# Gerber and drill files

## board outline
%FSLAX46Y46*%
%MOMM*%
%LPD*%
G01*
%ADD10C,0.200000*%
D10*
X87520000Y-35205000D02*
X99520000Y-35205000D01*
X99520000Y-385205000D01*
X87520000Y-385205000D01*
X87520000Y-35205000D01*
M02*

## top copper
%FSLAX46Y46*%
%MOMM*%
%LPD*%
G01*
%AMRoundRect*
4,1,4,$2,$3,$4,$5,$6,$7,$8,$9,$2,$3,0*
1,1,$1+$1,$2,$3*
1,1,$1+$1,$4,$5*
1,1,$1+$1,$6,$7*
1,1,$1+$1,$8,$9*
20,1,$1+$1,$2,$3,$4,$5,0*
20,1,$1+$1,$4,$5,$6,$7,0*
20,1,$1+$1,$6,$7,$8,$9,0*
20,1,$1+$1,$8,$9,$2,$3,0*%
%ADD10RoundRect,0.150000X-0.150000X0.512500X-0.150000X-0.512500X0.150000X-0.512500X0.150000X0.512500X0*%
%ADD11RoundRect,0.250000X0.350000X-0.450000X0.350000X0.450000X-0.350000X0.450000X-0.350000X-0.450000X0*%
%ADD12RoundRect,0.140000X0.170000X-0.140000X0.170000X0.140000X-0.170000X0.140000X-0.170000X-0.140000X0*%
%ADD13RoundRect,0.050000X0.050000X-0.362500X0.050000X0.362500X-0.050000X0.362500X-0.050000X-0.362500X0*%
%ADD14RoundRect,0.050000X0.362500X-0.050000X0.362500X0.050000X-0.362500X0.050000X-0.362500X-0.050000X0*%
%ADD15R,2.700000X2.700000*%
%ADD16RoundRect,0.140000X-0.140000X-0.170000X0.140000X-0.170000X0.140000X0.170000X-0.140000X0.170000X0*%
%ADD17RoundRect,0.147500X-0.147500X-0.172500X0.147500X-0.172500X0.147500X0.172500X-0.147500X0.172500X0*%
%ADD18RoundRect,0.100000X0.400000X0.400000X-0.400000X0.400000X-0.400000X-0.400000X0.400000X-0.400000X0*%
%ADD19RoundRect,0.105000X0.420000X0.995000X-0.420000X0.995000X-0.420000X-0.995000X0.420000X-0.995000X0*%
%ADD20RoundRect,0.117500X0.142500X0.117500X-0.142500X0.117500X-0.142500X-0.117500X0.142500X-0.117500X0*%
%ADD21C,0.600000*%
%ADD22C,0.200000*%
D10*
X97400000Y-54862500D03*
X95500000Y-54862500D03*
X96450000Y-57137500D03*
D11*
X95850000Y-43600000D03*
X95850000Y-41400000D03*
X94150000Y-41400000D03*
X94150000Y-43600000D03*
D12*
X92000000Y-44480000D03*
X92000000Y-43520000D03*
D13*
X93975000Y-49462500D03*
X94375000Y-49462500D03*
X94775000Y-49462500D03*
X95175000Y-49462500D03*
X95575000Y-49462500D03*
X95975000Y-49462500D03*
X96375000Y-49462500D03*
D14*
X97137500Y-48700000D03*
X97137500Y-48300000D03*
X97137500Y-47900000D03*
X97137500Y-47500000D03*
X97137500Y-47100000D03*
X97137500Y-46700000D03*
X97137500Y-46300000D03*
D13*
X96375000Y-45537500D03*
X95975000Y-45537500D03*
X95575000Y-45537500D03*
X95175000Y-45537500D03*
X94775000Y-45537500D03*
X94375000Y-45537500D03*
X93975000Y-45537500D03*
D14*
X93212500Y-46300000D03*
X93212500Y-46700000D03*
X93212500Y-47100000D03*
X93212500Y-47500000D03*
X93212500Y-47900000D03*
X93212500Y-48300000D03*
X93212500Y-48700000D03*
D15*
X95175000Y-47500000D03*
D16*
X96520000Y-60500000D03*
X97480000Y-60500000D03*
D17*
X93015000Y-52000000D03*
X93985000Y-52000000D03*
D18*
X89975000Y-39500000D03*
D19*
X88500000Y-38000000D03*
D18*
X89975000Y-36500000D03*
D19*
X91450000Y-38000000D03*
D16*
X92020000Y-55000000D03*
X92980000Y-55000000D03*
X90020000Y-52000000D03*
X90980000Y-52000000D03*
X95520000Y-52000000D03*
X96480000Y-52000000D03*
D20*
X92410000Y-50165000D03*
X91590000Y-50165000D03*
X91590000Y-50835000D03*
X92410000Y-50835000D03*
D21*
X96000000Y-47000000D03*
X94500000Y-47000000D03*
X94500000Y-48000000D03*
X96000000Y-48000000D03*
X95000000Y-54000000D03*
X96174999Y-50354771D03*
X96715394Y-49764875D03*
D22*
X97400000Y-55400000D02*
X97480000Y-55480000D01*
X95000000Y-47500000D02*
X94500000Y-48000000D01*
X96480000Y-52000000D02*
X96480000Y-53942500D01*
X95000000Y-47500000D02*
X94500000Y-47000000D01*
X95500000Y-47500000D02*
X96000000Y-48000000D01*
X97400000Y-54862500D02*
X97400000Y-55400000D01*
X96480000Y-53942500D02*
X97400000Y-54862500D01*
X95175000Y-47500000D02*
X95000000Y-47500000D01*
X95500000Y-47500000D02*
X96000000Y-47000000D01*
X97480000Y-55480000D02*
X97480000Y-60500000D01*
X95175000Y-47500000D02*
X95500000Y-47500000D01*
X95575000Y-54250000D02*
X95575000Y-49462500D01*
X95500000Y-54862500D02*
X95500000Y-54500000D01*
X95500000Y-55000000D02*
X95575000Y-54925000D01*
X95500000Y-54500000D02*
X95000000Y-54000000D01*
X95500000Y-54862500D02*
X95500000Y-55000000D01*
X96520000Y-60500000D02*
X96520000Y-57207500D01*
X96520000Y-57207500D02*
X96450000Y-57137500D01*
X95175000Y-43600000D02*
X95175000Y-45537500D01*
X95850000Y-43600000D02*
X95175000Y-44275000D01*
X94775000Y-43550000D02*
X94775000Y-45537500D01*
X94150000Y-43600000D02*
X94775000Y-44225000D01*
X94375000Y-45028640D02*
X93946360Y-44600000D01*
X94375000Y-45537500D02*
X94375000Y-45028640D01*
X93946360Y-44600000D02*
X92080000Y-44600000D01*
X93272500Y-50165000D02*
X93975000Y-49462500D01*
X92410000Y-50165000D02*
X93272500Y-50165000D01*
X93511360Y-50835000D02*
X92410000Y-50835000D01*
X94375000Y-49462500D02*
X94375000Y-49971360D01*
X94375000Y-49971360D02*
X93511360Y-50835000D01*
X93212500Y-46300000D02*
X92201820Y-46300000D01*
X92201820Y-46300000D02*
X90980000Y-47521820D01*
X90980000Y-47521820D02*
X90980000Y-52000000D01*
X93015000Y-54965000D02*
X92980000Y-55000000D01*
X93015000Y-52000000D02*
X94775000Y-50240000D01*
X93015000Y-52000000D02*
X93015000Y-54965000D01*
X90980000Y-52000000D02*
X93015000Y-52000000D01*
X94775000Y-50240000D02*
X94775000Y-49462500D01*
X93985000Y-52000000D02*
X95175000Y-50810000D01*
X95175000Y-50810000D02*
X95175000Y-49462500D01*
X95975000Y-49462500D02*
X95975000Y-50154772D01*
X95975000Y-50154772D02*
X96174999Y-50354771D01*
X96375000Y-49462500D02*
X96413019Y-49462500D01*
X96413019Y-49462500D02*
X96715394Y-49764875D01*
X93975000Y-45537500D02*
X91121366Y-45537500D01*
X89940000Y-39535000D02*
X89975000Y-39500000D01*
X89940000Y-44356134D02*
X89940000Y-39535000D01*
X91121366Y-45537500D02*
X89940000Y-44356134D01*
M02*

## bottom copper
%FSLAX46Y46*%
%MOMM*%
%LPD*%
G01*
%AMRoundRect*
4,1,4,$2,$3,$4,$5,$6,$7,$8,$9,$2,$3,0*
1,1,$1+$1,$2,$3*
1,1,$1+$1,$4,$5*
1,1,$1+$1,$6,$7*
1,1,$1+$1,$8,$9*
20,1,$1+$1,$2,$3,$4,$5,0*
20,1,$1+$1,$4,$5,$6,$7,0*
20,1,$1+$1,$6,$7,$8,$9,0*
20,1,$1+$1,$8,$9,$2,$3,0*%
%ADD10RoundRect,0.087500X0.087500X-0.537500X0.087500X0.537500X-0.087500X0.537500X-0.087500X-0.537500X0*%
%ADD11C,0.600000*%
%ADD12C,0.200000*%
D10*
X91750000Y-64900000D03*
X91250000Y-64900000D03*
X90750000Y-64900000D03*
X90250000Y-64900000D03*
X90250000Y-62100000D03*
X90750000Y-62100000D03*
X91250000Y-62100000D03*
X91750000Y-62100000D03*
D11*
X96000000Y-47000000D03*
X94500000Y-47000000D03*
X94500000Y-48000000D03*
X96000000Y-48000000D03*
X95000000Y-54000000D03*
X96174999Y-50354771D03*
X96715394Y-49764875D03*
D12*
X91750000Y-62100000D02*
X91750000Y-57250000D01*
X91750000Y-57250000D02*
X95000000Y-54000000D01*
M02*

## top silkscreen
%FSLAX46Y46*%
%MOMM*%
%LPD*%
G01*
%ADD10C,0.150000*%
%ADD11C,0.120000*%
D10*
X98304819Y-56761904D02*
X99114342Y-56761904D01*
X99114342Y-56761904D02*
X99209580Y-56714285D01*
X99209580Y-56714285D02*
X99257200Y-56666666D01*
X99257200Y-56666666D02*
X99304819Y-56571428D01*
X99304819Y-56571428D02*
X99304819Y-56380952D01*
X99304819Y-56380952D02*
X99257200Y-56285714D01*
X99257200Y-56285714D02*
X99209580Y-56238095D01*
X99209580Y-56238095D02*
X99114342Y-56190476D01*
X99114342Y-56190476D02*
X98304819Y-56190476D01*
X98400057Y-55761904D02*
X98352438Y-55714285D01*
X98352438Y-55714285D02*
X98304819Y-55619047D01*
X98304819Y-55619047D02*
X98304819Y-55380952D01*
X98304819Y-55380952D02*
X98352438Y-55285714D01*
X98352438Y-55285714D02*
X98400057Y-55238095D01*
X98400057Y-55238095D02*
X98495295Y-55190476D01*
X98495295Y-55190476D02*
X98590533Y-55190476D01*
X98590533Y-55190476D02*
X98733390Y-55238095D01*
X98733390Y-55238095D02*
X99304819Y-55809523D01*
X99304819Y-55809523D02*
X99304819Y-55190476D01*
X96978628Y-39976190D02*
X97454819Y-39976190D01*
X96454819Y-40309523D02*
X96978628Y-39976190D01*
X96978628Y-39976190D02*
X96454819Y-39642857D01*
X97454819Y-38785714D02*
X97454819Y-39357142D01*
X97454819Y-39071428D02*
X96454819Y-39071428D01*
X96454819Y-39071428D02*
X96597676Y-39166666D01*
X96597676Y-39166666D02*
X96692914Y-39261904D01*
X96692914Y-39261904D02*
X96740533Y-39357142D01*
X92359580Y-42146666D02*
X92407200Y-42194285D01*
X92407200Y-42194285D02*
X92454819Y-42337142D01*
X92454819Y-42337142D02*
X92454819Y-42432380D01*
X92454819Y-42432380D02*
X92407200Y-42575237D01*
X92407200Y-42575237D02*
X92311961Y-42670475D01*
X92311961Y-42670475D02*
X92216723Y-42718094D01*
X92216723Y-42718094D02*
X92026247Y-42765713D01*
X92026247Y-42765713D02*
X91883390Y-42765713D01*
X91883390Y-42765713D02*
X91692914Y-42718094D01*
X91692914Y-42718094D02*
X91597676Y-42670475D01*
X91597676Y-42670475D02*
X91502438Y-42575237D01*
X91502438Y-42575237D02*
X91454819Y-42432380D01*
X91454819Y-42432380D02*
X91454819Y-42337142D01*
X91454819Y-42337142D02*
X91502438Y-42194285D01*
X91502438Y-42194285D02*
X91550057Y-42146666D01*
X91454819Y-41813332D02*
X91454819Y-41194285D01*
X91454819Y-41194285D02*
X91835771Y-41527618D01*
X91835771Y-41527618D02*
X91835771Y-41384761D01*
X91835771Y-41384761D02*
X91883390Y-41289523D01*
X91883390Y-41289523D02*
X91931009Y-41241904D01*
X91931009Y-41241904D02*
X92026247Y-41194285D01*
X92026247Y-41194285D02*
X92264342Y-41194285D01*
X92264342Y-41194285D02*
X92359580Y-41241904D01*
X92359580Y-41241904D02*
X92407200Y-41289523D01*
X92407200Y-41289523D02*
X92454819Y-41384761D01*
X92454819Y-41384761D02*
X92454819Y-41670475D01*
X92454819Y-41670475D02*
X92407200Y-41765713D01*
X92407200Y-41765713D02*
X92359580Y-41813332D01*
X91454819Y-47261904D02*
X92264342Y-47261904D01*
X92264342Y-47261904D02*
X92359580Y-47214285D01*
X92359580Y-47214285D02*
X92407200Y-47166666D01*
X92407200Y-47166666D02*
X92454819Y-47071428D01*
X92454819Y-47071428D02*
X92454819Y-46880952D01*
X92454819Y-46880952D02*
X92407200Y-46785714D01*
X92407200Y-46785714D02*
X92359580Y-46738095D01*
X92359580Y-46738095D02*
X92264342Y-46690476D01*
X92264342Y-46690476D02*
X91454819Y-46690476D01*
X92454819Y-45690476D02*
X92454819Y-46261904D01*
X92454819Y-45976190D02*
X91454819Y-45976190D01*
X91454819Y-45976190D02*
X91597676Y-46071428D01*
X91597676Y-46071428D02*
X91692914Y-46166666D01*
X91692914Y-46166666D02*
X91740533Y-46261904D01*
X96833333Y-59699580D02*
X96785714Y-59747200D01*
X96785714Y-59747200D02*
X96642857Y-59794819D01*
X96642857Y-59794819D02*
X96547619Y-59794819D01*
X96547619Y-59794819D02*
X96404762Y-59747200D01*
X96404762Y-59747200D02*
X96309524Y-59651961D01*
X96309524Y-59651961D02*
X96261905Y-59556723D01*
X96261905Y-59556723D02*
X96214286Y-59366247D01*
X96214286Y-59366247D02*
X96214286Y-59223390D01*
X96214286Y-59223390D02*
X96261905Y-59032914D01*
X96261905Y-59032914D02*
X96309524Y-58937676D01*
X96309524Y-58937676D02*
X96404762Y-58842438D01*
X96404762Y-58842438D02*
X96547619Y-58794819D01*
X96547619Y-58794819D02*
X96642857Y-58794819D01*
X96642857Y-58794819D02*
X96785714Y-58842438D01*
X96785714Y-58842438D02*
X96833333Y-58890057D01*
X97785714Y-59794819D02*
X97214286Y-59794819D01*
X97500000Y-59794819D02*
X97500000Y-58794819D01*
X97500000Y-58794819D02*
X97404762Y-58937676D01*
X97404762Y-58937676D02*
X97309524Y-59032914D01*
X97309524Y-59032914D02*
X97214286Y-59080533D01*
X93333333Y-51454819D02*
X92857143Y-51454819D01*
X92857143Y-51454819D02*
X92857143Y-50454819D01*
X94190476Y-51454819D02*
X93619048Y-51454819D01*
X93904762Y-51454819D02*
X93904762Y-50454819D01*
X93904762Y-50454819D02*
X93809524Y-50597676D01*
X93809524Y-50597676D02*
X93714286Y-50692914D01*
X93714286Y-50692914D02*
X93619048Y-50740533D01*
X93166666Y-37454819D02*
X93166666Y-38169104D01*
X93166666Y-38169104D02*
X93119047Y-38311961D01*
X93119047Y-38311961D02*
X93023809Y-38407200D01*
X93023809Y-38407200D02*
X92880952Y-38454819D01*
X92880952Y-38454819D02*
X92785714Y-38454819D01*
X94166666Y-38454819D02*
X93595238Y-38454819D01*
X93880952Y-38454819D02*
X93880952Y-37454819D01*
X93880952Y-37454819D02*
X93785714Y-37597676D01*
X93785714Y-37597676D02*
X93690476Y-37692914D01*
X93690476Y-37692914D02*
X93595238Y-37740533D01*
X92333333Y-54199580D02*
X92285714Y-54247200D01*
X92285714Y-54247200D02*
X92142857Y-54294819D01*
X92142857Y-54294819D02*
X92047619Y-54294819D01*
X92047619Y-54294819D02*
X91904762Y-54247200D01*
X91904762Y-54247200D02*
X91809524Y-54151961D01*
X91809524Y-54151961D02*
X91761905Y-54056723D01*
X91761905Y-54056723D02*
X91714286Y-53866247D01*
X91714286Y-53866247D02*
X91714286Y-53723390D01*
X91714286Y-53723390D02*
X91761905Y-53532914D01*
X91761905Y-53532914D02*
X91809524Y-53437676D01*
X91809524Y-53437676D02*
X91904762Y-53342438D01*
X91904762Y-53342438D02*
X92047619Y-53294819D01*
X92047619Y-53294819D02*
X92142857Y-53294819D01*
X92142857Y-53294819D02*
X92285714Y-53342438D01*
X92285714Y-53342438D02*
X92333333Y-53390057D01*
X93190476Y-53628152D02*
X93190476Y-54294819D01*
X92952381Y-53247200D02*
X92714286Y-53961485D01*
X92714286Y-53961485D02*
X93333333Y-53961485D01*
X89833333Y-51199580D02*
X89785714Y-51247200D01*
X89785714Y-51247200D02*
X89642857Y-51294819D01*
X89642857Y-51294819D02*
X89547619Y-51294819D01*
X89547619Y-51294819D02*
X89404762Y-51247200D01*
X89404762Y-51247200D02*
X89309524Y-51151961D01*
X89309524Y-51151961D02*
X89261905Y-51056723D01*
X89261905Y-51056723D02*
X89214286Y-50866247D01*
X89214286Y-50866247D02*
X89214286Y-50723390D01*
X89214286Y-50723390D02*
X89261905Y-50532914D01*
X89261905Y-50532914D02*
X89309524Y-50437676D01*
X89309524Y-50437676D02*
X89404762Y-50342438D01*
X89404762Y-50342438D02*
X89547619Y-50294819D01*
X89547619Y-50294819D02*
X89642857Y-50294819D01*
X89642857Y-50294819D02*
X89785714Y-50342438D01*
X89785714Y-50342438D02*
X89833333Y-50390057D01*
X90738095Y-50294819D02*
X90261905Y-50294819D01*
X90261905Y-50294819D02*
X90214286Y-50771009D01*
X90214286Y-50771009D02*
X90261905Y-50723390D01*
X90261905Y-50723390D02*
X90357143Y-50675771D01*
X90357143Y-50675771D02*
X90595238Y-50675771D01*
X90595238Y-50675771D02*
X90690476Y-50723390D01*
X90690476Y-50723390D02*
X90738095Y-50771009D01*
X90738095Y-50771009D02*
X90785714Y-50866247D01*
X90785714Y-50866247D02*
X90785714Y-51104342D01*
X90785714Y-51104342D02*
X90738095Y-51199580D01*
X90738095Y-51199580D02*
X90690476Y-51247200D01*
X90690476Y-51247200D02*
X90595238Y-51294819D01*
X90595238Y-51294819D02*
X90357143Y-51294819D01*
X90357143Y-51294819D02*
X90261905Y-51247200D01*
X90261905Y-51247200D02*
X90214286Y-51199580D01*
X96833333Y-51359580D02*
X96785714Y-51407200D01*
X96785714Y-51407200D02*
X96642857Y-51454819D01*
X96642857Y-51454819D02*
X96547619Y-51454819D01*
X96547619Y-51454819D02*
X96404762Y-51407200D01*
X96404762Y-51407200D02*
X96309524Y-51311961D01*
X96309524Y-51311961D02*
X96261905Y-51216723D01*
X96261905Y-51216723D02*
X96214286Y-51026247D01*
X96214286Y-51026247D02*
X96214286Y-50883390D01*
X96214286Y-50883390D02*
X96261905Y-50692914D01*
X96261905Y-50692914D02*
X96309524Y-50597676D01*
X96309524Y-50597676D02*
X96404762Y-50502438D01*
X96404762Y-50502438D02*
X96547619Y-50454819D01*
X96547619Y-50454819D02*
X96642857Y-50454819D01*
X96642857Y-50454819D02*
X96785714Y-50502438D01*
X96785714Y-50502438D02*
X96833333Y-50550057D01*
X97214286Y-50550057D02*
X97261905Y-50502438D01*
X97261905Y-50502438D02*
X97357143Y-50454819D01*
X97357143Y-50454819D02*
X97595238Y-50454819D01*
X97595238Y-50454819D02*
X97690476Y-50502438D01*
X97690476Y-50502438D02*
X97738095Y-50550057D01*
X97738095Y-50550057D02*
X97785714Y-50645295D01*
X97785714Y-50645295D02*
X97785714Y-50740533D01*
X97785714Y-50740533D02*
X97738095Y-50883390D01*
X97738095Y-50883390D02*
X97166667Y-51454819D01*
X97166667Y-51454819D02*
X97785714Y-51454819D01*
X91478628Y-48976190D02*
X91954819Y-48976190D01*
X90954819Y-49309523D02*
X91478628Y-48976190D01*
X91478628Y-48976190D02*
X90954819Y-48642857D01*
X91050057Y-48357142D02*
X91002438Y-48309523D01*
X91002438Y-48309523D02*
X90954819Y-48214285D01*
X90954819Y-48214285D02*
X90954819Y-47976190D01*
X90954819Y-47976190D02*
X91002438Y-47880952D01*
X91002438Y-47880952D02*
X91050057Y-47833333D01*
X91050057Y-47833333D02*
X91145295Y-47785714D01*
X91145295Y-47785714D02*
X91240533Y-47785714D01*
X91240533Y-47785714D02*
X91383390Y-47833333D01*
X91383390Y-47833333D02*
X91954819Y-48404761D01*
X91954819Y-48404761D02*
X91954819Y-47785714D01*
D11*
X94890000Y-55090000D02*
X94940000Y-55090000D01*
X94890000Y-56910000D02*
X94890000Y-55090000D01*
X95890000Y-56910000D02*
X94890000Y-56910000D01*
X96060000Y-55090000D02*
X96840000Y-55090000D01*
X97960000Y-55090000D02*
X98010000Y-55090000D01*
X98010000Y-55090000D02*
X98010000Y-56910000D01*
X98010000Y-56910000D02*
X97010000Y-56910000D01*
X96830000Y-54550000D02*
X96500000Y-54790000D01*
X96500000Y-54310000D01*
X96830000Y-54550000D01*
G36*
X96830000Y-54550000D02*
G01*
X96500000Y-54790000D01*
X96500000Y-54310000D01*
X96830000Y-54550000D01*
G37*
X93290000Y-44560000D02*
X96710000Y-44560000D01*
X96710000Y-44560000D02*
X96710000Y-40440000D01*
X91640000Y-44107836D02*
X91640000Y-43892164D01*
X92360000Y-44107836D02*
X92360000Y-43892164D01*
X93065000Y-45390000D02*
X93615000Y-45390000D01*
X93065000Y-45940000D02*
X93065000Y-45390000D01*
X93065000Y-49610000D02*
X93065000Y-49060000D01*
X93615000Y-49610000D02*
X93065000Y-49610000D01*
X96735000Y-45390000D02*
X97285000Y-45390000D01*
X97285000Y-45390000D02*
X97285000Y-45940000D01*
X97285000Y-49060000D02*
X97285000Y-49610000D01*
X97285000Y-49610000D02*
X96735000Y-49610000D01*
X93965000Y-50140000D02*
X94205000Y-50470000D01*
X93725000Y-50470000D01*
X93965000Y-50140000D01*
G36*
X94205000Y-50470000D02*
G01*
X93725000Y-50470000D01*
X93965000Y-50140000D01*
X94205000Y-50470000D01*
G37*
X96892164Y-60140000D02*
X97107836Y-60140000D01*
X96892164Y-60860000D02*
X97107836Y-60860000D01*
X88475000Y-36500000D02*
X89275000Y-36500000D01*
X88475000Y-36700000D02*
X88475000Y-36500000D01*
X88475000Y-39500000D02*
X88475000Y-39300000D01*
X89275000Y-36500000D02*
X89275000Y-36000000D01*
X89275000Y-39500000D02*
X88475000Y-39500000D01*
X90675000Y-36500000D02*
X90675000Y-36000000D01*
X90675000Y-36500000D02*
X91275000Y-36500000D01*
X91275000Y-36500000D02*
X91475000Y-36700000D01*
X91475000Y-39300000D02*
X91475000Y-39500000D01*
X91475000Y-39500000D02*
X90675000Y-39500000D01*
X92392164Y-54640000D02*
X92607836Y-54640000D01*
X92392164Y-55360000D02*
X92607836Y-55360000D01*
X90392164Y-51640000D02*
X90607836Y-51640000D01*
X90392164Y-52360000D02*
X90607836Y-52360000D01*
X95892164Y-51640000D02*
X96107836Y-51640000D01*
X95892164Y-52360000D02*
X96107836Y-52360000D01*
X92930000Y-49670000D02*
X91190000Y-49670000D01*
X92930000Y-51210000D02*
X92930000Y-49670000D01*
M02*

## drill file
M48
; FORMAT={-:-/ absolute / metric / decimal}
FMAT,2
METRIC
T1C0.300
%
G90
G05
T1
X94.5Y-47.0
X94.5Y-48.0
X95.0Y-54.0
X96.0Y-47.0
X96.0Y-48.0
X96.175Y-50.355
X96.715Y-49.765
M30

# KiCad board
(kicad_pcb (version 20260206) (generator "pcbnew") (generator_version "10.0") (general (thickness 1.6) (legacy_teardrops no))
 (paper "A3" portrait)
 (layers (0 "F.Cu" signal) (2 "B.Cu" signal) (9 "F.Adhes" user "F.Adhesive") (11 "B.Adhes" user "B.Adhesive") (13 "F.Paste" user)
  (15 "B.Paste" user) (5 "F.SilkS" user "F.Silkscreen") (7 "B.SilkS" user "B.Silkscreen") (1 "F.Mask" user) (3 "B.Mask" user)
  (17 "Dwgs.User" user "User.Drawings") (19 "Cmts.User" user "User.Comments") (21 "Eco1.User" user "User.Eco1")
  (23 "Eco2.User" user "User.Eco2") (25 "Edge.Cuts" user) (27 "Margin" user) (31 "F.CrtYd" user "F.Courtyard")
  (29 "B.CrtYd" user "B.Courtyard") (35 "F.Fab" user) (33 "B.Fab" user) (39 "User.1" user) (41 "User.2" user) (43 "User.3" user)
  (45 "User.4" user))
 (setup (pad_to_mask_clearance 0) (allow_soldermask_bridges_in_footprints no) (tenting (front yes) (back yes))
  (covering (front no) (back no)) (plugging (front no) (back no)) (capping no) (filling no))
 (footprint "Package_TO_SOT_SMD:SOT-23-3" (layer "F.Cu") (at 96.45 56 -90)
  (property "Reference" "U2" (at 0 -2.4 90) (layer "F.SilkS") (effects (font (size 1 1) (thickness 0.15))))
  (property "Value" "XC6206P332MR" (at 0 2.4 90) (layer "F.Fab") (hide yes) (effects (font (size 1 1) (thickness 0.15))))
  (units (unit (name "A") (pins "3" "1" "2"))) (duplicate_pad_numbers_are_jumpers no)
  (fp_line (start -0.91 1.56) (end -0.91 1.51) (stroke (width 0.12) (type solid)) (layer "F.SilkS"))
  (fp_line (start 0.91 1.56) (end -0.91 1.56) (stroke (width 0.12) (type solid)) (layer "F.SilkS"))
  (fp_line (start 0.91 0.56) (end 0.91 1.56) (stroke (width 0.12) (type solid)) (layer "F.SilkS"))
  (fp_line (start -0.91 0.39) (end -0.91 -0.39) (stroke (width 0.12) (type solid)) (layer "F.SilkS"))
  (fp_line (start -0.91 -1.51) (end -0.91 -1.56) (stroke (width 0.12) (type solid)) (layer "F.SilkS"))
  (fp_line (start -0.91 -1.56) (end 0.91 -1.56) (stroke (width 0.12) (type solid)) (layer "F.SilkS"))
  (fp_line (start 0.91 -1.56) (end 0.91 -0.56) (stroke (width 0.12) (type solid)) (layer "F.SilkS"))
  (fp_poly (pts (xy -1.45 -0.38) (xy -1.21 -0.05) (xy -1.69 -0.05)) (stroke (width 0.12) (type solid)) (fill yes) (layer "F.SilkS"))
  (pad "1" smd roundrect (at -1.1375 -0.95 270) (size 1.325 0.6) (layers "F.Cu" "F.Mask" "F.Paste") (roundrect_rratio 0.25) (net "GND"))
  (pad "2" smd roundrect (at -1.1375 0.95 270) (size 1.325 0.6) (layers "F.Cu" "F.Mask" "F.Paste") (roundrect_rratio 0.25) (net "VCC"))
  (pad "3" smd roundrect (at 1.1375 0 270) (size 1.325 0.6) (layers "F.Cu" "F.Mask" "F.Paste") (roundrect_rratio 0.25) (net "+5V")))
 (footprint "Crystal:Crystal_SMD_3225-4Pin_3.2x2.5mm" (layer "F.Cu") (at 95 42.5 90)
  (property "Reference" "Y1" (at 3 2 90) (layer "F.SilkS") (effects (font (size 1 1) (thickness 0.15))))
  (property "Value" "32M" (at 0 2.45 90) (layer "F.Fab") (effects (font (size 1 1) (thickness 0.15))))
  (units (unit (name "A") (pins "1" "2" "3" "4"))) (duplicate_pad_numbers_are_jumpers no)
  (fp_line (start -2.06 -1.71) (end -2.06 1.71) (stroke (width 0.12) (type solid)) (layer "F.SilkS"))
  (fp_line (start -2.06 1.71) (end 2.06 1.71) (stroke (width 0.12) (type solid)) (layer "F.SilkS"))
  (pad "1" smd roundrect (at -1.1 0.85 90) (size 1.4 1.2) (layers "F.Cu" "F.Mask" "F.Paste") (roundrect_rratio 0.208333)
   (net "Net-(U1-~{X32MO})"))
  (pad "2" smd roundrect (at 1.1 0.85 90) (size 1.4 1.2) (layers "F.Cu" "F.Mask" "F.Paste") (roundrect_rratio 0.208333) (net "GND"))
  (pad "3" smd roundrect (at 1.1 -0.85 90) (size 1.4 1.2) (layers "F.Cu" "F.Mask" "F.Paste") (roundrect_rratio 0.208333) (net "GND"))
  (pad "4" smd roundrect (at -1.1 -0.85 90) (size 1.4 1.2) (layers "F.Cu" "F.Mask" "F.Paste") (roundrect_rratio 0.208333)
   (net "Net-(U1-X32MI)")))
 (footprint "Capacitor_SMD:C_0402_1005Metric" (layer "F.Cu") (at 92 44 90)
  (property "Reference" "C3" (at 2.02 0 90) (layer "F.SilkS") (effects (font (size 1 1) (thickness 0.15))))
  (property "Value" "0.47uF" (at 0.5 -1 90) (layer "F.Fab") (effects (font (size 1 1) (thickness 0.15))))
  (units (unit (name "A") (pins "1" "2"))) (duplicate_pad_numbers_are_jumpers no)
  (fp_line (start -0.107836 -0.36) (end 0.107836 -0.36) (stroke (width 0.12) (type solid)) (layer "F.SilkS"))
  (fp_line (start -0.107836 0.36) (end 0.107836 0.36) (stroke (width 0.12) (type solid)) (layer "F.SilkS"))
  (pad "1" smd roundrect (at -0.48 0 90) (size 0.56 0.62) (layers "F.Cu" "F.Mask" "F.Paste") (roundrect_rratio 0.25) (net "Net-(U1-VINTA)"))
  (pad "2" smd roundrect (at 0.48 0 90) (size 0.56 0.62) (layers "F.Cu" "F.Mask" "F.Paste") (roundrect_rratio 0.25) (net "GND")))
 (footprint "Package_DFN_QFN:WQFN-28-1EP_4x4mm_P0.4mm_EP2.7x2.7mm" (layer "F.Cu") (at 95.175 47.5 90)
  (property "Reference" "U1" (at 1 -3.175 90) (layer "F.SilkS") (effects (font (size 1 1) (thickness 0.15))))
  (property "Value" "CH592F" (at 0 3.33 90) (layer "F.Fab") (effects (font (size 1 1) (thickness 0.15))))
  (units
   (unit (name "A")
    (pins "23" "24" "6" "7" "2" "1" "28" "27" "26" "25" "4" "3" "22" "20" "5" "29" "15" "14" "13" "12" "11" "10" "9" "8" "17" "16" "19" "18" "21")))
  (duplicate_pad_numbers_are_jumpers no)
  (fp_line (start 2.11 -2.11) (end 2.11 -1.56) (stroke (width 0.12) (type solid)) (layer "F.SilkS"))
  (fp_line (start 1.56 -2.11) (end 2.11 -2.11) (stroke (width 0.12) (type solid)) (layer "F.SilkS"))
  (fp_line (start -2.11 -2.11) (end -1.56 -2.11) (stroke (width 0.12) (type solid)) (layer "F.SilkS"))
  (fp_line (start -2.11 -1.56) (end -2.11 -2.11) (stroke (width 0.12) (type solid)) (layer "F.SilkS"))
  (fp_line (start 2.11 1.56) (end 2.11 2.11) (stroke (width 0.12) (type solid)) (layer "F.SilkS"))
  (fp_line (start 2.11 2.11) (end 1.56 2.11) (stroke (width 0.12) (type solid)) (layer "F.SilkS"))
  (fp_line (start -1.56 2.11) (end -2.11 2.11) (stroke (width 0.12) (type solid)) (layer "F.SilkS"))
  (fp_line (start -2.11 2.11) (end -2.11 1.56) (stroke (width 0.12) (type solid)) (layer "F.SilkS"))
  (fp_poly (pts (xy -2.64 -1.21) (xy -2.97 -0.97) (xy -2.97 -1.45)) (stroke (width 0.12) (type solid)) (fill yes) (layer "F.SilkS"))
  (pad "" smd roundrect (at -0.675 -0.675 90) (size 1.09 1.09) (layers "F.Paste") (roundrect_rratio 0.229358))
  (pad "" smd roundrect (at -0.675 0.675 90) (size 1.09 1.09) (layers "F.Paste") (roundrect_rratio 0.229358))
  (pad "" smd roundrect (at 0.675 -0.675 90) (size 1.09 1.09) (layers "F.Paste") (roundrect_rratio 0.229358))
  (pad "" smd roundrect (at 0.675 0.675 90) (size 1.09 1.09) (layers "F.Paste") (roundrect_rratio 0.229358))
  (pad "1" smd roundrect (at -1.9625 -1.2 90) (size 0.825 0.2) (layers "F.Cu" "F.Mask" "F.Paste") (roundrect_rratio 0.25)
   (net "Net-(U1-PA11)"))
  (pad "2" smd roundrect (at -1.9625 -0.8 90) (size 0.825 0.2) (layers "F.Cu" "F.Mask" "F.Paste") (roundrect_rratio 0.25)
   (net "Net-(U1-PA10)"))
  (pad "3" smd roundrect (at -1.9625 -0.4 90) (size 0.825 0.2) (layers "F.Cu" "F.Mask" "F.Paste") (roundrect_rratio 0.25)
   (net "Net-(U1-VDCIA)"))
  (pad "4" smd roundrect (at -1.9625 0 90) (size 0.825 0.2) (layers "F.Cu" "F.Mask" "F.Paste") (roundrect_rratio 0.25) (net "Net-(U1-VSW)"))
  (pad "5" smd roundrect (at -1.9625 0.4 90) (size 0.825 0.2) (layers "F.Cu" "F.Mask" "F.Paste") (roundrect_rratio 0.25) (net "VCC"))
  (pad "6" smd roundrect (at -1.9625 0.8 90) (size 0.825 0.2) (layers "F.Cu" "F.Mask" "F.Paste") (roundrect_rratio 0.25)
   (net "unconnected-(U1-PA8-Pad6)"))
  (pad "7" smd roundrect (at -1.9625 1.2 90) (size 0.825 0.2) (layers "F.Cu" "F.Mask" "F.Paste") (roundrect_rratio 0.25)
   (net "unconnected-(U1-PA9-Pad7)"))
  (pad "8" smd roundrect (at -1.2 1.9625 90) (size 0.2 0.825) (layers "F.Cu" "F.Mask" "F.Paste") (roundrect_rratio 0.25)
   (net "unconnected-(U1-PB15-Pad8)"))
  (pad "9" smd roundrect (at -0.8 1.9625 90) (size 0.2 0.825) (layers "F.Cu" "F.Mask" "F.Paste") (roundrect_rratio 0.25)
   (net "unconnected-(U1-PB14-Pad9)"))
  (pad "10" smd roundrect (at -0.4 1.9625 90) (size 0.2 0.825) (layers "F.Cu" "F.Mask" "F.Paste") (roundrect_rratio 0.25)
   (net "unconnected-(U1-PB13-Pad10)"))
  (pad "11" smd roundrect (at 0 1.9625 90) (size 0.2 0.825) (layers "F.Cu" "F.Mask" "F.Paste") (roundrect_rratio 0.25)
   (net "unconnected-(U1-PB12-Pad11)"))
  (pad "12" smd roundrect (at 0.4 1.9625 90) (size 0.2 0.825) (layers "F.Cu" "F.Mask" "F.Paste") (roundrect_rratio 0.25)
   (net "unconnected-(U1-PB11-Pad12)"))
  (pad "13" smd roundrect (at 0.8 1.9625 90) (size 0.2 0.825) (layers "F.Cu" "F.Mask" "F.Paste") (roundrect_rratio 0.25)
   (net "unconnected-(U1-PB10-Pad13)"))
  (pad "14" smd roundrect (at 1.2 1.9625 90) (size 0.2 0.825) (layers "F.Cu" "F.Mask" "F.Paste") (roundrect_rratio 0.25)
   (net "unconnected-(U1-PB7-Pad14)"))
  (pad "15" smd roundrect (at 1.9625 1.2 90) (size 0.825 0.2) (layers "F.Cu" "F.Mask" "F.Paste") (roundrect_rratio 0.25)
   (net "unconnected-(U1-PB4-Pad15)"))
  (pad "16" smd roundrect (at 1.9625 0.8 90) (size 0.825 0.2) (layers "F.Cu" "F.Mask" "F.Paste") (roundrect_rratio 0.25)
   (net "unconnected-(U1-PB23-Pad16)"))
  (pad "17" smd roundrect (at 1.9625 0.4 90) (size 0.825 0.2) (layers "F.Cu" "F.Mask" "F.Paste") (roundrect_rratio 0.25)
   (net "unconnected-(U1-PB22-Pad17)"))
  (pad "18" smd roundrect (at 1.9625 0 90) (size 0.825 0.2) (layers "F.Cu" "F.Mask" "F.Paste") (roundrect_rratio 0.25)
   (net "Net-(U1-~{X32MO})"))
  (pad "19" smd roundrect (at 1.9625 -0.4 90) (size 0.825 0.2) (layers "F.Cu" "F.Mask" "F.Paste") (roundrect_rratio 0.25)
   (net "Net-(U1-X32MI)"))
  (pad "20" smd roundrect (at 1.9625 -0.8 90) (size 0.825 0.2) (layers "F.Cu" "F.Mask" "F.Paste") (roundrect_rratio 0.25)
   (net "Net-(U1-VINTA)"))
  (pad "21" smd roundrect (at 1.9625 -1.2 90) (size 0.825 0.2) (layers "F.Cu" "F.Mask" "F.Paste") (roundrect_rratio 0.25)
   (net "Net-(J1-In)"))
  (pad "22" smd roundrect (at 1.2 -1.9625 90) (size 0.2 0.825) (layers "F.Cu" "F.Mask" "F.Paste") (roundrect_rratio 0.25)
   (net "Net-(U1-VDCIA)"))
  (pad "23" smd roundrect (at 0.8 -1.9625 90) (size 0.2 0.825) (layers "F.Cu" "F.Mask" "F.Paste") (roundrect_rratio 0.25)
   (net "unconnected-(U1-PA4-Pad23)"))
  (pad "24" smd roundrect (at 0.4 -1.9625 90) (size 0.2 0.825) (layers "F.Cu" "F.Mask" "F.Paste") (roundrect_rratio 0.25)
   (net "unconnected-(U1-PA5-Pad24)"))
  (pad "25" smd roundrect (at 0 -1.9625 90) (size 0.2 0.825) (layers "F.Cu" "F.Mask" "F.Paste") (roundrect_rratio 0.25)
   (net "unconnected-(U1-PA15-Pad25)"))
  (pad "26" smd roundrect (at -0.4 -1.9625 90) (size 0.2 0.825) (layers "F.Cu" "F.Mask" "F.Paste") (roundrect_rratio 0.25)
   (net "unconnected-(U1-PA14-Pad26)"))
  (pad "27" smd roundrect (at -0.8 -1.9625 90) (size 0.2 0.825) (layers "F.Cu" "F.Mask" "F.Paste") (roundrect_rratio 0.25)
   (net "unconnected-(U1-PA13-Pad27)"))
  (pad "28" smd roundrect (at -1.2 -1.9625 90) (size 0.2 0.825) (layers "F.Cu" "F.Mask" "F.Paste") (roundrect_rratio 0.25)
   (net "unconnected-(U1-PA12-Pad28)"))
  (pad "29" smd rect (at 0 0 90) (size 2.7 2.7) (layers "F.Cu" "F.Mask") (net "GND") (zone_connect 2)))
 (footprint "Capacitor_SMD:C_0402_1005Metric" (layer "F.Cu") (at 97 60.5)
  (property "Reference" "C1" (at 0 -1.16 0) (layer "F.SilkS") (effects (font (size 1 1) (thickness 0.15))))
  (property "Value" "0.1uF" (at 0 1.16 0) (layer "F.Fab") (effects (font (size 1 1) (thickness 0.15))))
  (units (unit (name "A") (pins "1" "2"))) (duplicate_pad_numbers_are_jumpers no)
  (fp_line (start -0.107836 -0.36) (end 0.107836 -0.36) (stroke (width 0.12) (type solid)) (layer "F.SilkS"))
  (fp_line (start -0.107836 0.36) (end 0.107836 0.36) (stroke (width 0.12) (type solid)) (layer "F.SilkS"))
  (pad "1" smd roundrect (at -0.48 0) (size 0.56 0.62) (layers "F.Cu" "F.Mask" "F.Paste") (roundrect_rratio 0.25) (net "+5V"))
  (pad "2" smd roundrect (at 0.48 0) (size 0.56 0.62) (layers "F.Cu" "F.Mask" "F.Paste") (roundrect_rratio 0.25) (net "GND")))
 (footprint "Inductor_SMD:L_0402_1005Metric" (layer "F.Cu") (at 93.5 52)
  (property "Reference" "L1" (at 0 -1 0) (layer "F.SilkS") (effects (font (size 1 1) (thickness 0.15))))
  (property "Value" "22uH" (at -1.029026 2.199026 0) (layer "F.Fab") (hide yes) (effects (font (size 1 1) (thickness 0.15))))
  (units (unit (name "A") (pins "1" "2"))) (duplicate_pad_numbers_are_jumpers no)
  (pad "1" smd roundrect (at -0.485 0) (size 0.59 0.64) (layers "F.Cu" "F.Mask" "F.Paste") (roundrect_rratio 0.25) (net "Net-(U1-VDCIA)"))
  (pad "2" smd roundrect (at 0.485 0) (size 0.59 0.64) (layers "F.Cu" "F.Mask" "F.Paste") (roundrect_rratio 0.25) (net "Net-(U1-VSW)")))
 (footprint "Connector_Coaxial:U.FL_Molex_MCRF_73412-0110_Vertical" (layer "F.Cu") (at 89.975 38)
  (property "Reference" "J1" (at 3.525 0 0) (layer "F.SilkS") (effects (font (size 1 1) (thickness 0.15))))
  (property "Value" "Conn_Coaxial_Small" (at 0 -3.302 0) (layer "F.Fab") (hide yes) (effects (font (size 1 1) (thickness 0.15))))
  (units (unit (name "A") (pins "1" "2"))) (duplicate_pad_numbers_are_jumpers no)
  (fp_line (start -1.5 -1.5) (end -0.7 -1.5) (stroke (width 0.12) (type solid)) (layer "F.SilkS"))
  (fp_line (start -1.5 -1.3) (end -1.5 -1.5) (stroke (width 0.12) (type solid)) (layer "F.SilkS"))
  (fp_line (start -1.5 1.5) (end -1.5 1.3) (stroke (width 0.12) (type solid)) (layer "F.SilkS"))
  (fp_line (start -0.7 -1.5) (end -0.7 -2) (stroke (width 0.12) (type solid)) (layer "F.SilkS"))
  (fp_line (start -0.7 1.5) (end -1.5 1.5) (stroke (width 0.12) (type solid)) (layer "F.SilkS"))
  (fp_line (start 0.7 -1.5) (end 0.7 -2) (stroke (width 0.12) (type solid)) (layer "F.SilkS"))
  (fp_line (start 0.7 -1.5) (end 1.3 -1.5) (stroke (width 0.12) (type solid)) (layer "F.SilkS"))
  (fp_line (start 1.3 -1.5) (end 1.5 -1.3) (stroke (width 0.12) (type solid)) (layer "F.SilkS"))
  (fp_line (start 1.5 1.3) (end 1.5 1.5) (stroke (width 0.12) (type solid)) (layer "F.SilkS"))
  (fp_line (start 1.5 1.5) (end 0.7 1.5) (stroke (width 0.12) (type solid)) (layer "F.SilkS"))
  (pad "1" smd roundrect (at 0 1.5 180) (size 1 1) (layers "F.Cu" "F.Mask" "F.Paste") (roundrect_rratio 0.1) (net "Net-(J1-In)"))
  (pad "2" smd roundrect (at -1.475 0 180) (size 1.05 2.2) (layers "F.Cu" "F.Mask" "F.Paste") (roundrect_rratio 0.1) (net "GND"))
  (pad "2" smd roundrect (at 0 -1.5 180) (size 1 1) (layers "F.Cu" "F.Mask" "F.Paste") (roundrect_rratio 0.1) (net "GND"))
  (pad "2" smd roundrect (at 1.475 0 180) (size 1.05 2.2) (layers "F.Cu" "F.Mask" "F.Paste") (roundrect_rratio 0.1) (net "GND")))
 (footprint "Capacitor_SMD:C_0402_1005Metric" (layer "F.Cu") (at 92.5 55)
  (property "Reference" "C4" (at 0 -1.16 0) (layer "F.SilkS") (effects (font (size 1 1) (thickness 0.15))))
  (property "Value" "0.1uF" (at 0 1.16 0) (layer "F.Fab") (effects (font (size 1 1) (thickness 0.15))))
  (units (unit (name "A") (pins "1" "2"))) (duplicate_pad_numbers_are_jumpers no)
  (fp_line (start -0.107836 -0.36) (end 0.107836 -0.36) (stroke (width 0.12) (type solid)) (layer "F.SilkS"))
  (fp_line (start -0.107836 0.36) (end 0.107836 0.36) (stroke (width 0.12) (type solid)) (layer "F.SilkS"))
  (pad "1" smd roundrect (at -0.48 0) (size 0.56 0.62) (layers "F.Cu" "F.Mask" "F.Paste") (roundrect_rratio 0.25) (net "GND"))
  (pad "2" smd roundrect (at 0.48 0) (size 0.56 0.62) (layers "F.Cu" "F.Mask" "F.Paste") (roundrect_rratio 0.25) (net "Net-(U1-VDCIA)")))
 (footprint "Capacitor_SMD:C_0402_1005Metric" (layer "F.Cu") (at 90.5 52)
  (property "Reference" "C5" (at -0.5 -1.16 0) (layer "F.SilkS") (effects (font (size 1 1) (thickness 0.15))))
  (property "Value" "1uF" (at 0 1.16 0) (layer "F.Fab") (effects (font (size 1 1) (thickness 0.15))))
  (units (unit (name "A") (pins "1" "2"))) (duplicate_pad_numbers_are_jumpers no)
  (fp_line (start -0.107836 -0.36) (end 0.107836 -0.36) (stroke (width 0.12) (type solid)) (layer "F.SilkS"))
  (fp_line (start -0.107836 0.36) (end 0.107836 0.36) (stroke (width 0.12) (type solid)) (layer "F.SilkS"))
  (pad "1" smd roundrect (at -0.48 0) (size 0.56 0.62) (layers "F.Cu" "F.Mask" "F.Paste") (roundrect_rratio 0.25) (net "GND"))
  (pad "2" smd roundrect (at 0.48 0) (size 0.56 0.62) (layers "F.Cu" "F.Mask" "F.Paste") (roundrect_rratio 0.25) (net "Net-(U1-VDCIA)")))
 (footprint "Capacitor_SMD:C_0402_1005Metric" (layer "F.Cu") (at 96 52)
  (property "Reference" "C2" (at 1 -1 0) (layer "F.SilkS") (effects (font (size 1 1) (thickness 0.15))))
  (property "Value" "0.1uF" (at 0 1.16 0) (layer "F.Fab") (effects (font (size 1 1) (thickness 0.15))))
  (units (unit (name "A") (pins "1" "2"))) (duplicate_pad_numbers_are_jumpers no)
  (fp_line (start -0.107836 -0.36) (end 0.107836 -0.36) (stroke (width 0.12) (type solid)) (layer "F.SilkS"))
  (fp_line (start -0.107836 0.36) (end 0.107836 0.36) (stroke (width 0.12) (type solid)) (layer "F.SilkS"))
  (pad "1" smd roundrect (at -0.48 0) (size 0.56 0.62) (layers "F.Cu" "F.Mask" "F.Paste") (roundrect_rratio 0.25) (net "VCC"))
  (pad "2" smd roundrect (at 0.48 0) (size 0.56 0.62) (layers "F.Cu" "F.Mask" "F.Paste") (roundrect_rratio 0.25) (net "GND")))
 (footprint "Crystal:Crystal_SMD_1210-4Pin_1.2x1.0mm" (layer "F.Cu") (at 92 50.5 -90)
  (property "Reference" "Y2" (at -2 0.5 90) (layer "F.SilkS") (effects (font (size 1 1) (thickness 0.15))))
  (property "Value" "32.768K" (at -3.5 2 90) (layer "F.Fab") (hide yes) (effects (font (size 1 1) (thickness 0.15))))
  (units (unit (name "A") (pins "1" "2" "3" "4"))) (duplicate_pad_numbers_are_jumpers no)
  (fp_line (start -0.83 -0.93) (end -0.83 0.81) (stroke (width 0.12) (type solid)) (layer "F.SilkS"))
  (fp_line (start 0.71 -0.93) (end -0.83 -0.93) (stroke (width 0.12) (type solid)) (layer "F.SilkS"))
  (pad "1" smd roundrect (at -0.335 -0.41 180) (size 0.52 0.47) (layers "F.Cu" "F.Mask" "F.Paste") (roundrect_rratio 0.25)
   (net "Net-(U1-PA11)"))
  (pad "2" smd roundrect (at -0.335 0.41 180) (size 0.52 0.47) (layers "F.Cu" "F.Mask" "F.Paste") (roundrect_rratio 0.25) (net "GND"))
  (pad "3" smd roundrect (at 0.335 0.41 180) (size 0.52 0.47) (layers "F.Cu" "F.Mask" "F.Paste") (roundrect_rratio 0.25) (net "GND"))
  (pad "4" smd roundrect (at 0.335 -0.41 180) (size 0.52 0.47) (layers "F.Cu" "F.Mask" "F.Paste") (roundrect_rratio 0.25)
   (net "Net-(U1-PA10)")))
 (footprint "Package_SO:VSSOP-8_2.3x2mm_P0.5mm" (layer "B.Cu") (at 91 63.5 90)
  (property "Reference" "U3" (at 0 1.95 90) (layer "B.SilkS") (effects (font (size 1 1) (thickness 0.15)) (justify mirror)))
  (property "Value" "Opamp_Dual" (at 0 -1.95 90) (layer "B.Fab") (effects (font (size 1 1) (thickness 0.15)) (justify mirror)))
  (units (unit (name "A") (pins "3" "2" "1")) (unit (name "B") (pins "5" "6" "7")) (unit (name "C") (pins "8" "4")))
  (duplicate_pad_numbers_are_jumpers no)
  (pad "1" smd roundrect (at -1.4 0.75 90) (size 1.25 0.35) (layers "B.Cu" "B.Mask" "B.Paste") (roundrect_rratio 0.25)
   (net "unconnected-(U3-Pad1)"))
  (pad "2" smd roundrect (at -1.4 0.25 90) (size 1.25 0.35) (layers "B.Cu" "B.Mask" "B.Paste") (roundrect_rratio 0.25)
   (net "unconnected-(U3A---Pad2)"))
  (pad "3" smd roundrect (at -1.4 -0.25 90) (size 1.25 0.35) (layers "B.Cu" "B.Mask" "B.Paste") (roundrect_rratio 0.25)
   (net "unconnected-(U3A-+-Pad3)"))
  (pad "4" smd roundrect (at -1.4 -0.75 90) (size 1.25 0.35) (layers "B.Cu" "B.Mask" "B.Paste") (roundrect_rratio 0.25) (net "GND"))
  (pad "5" smd roundrect (at 1.4 -0.75 90) (size 1.25 0.35) (layers "B.Cu" "B.Mask" "B.Paste") (roundrect_rratio 0.25)
   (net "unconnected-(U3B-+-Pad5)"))
  (pad "6" smd roundrect (at 1.4 -0.25 90) (size 1.25 0.35) (layers "B.Cu" "B.Mask" "B.Paste") (roundrect_rratio 0.25)
   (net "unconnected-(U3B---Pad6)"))
  (pad "7" smd roundrect (at 1.4 0.25 90) (size 1.25 0.35) (layers "B.Cu" "B.Mask" "B.Paste") (roundrect_rratio 0.25)
   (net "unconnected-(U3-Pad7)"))
  (pad "8" smd roundrect (at 1.4 0.75 90) (size 1.25 0.35) (layers "B.Cu" "B.Mask" "B.Paste") (roundrect_rratio 0.25) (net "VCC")))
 (gr_rect (start 87.52 35.205) (end 99.52 385.205) (stroke (width 0.2) (type solid)) (fill no) (layer "Edge.Cuts"))
 (segment (start 97.4 55.4) (end 97.48 55.48) (width 0.2) (layer "F.Cu") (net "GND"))
 (segment (start 95 47.5) (end 94.5 48) (width 0.2) (layer "F.Cu") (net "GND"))
 (segment (start 96.48 52) (end 96.48 53.9425) (width 0.2) (layer "F.Cu") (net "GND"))
 (segment (start 95 47.5) (end 94.5 47) (width 0.2) (layer "F.Cu") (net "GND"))
 (segment (start 95.5 47.5) (end 96 48) (width 0.2) (layer "F.Cu") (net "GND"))
 (segment (start 97.4 54.8625) (end 97.4 55.4) (width 0.2) (layer "F.Cu") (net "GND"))
 (segment (start 96.48 53.9425) (end 97.4 54.8625) (width 0.2) (layer "F.Cu") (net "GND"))
 (segment (start 95.175 47.5) (end 95 47.5) (width 0.2) (layer "F.Cu") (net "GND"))
 (segment (start 95.5 47.5) (end 96 47) (width 0.2) (layer "F.Cu") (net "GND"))
 (segment (start 97.48 55.48) (end 97.48 60.5) (width 0.2) (layer "F.Cu") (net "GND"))
 (segment (start 95.175 47.5) (end 95.5 47.5) (width 0.2) (layer "F.Cu") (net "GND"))
 (via (at 96 47) (size 0.6) (drill 0.3) (layers "F.Cu" "B.Cu") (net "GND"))
 (via (at 94.5 47) (size 0.6) (drill 0.3) (layers "F.Cu" "B.Cu") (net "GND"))
 (via (at 94.5 48) (size 0.6) (drill 0.3) (layers "F.Cu" "B.Cu") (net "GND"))
 (via (at 96 48) (size 0.6) (drill 0.3) (layers "F.Cu" "B.Cu") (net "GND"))
 (segment (start 95.575 54.25) (end 95.575 49.4625) (width 0.2) (layer "F.Cu") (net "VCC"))
 (segment (start 95.5 54.8625) (end 95.5 54.5) (width 0.2) (layer "F.Cu") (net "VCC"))
 (segment (start 95.5 55) (end 95.575 54.925) (width 0.2) (layer "F.Cu") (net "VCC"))
 (segment (start 95.5 54.5) (end 95 54) (width 0.2) (layer "F.Cu") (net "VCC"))
 (segment (start 95.5 54.8625) (end 95.5 55) (width 0.2) (layer "F.Cu") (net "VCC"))
 (via (at 95 54) (size 0.6) (drill 0.3) (layers "F.Cu" "B.Cu") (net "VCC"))
 (segment (start 91.75 62.1) (end 91.75 57.25) (width 0.2) (layer "B.Cu") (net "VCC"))
 (segment (start 91.75 57.25) (end 95 54) (width 0.2) (layer "B.Cu") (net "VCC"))
 (segment (start 96.52 60.5) (end 96.52 57.2075) (width 0.2) (layer "F.Cu") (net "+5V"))
 (segment (start 96.52 57.2075) (end 96.45 57.1375) (width 0.2) (layer "F.Cu") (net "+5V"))
 (segment (start 95.175 43.6) (end 95.175 45.5375) (width 0.2) (layer "F.Cu") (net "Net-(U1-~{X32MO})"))
 (segment (start 95.85 43.6) (end 95.175 44.275) (width 0.2) (layer "F.Cu") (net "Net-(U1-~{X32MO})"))
 (segment (start 94.775 43.55) (end 94.775 45.5375) (width 0.2) (layer "F.Cu") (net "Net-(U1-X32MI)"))
 (segment (start 94.15 43.6) (end 94.775 44.225) (width 0.2) (layer "F.Cu") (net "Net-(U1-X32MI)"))
 (segment (start 94.375 45.02864) (end 93.94636 44.6) (width 0.2) (layer "F.Cu") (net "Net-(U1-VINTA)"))
 (segment (start 94.375 45.5375) (end 94.375 45.02864) (width 0.2) (layer "F.Cu") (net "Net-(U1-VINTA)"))
 (segment (start 93.94636 44.6) (end 92.08 44.6) (width 0.2) (layer "F.Cu") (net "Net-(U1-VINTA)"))
 (segment (start 93.2725 50.165) (end 93.975 49.4625) (width 0.2) (layer "F.Cu") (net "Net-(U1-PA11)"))
 (segment (start 92.41 50.165) (end 93.2725 50.165) (width 0.2) (layer "F.Cu") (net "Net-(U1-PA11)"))
 (segment (start 93.51136 50.835) (end 92.41 50.835) (width 0.2) (layer "F.Cu") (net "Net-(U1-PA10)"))
 (segment (start 94.375 49.4625) (end 94.375 49.97136) (width 0.2) (layer "F.Cu") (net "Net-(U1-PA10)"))
 (segment (start 94.375 49.97136) (end 93.51136 50.835) (width 0.2) (layer "F.Cu") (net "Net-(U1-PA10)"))
 (segment (start 93.2125 46.3) (end 92.20182 46.3) (width 0.2) (layer "F.Cu") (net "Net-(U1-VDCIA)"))
 (segment (start 92.20182 46.3) (end 90.98 47.52182) (width 0.2) (layer "F.Cu") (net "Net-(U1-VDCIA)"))
 (segment (start 90.98 47.52182) (end 90.98 52) (width 0.2) (layer "F.Cu") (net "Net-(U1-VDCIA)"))
 (segment (start 93.015 54.965) (end 92.98 55) (width 0.2) (layer "F.Cu") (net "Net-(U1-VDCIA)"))
 (segment (start 93.015 52) (end 94.775 50.24) (width 0.2) (layer "F.Cu") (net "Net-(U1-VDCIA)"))
 (segment (start 93.015 52) (end 93.015 54.965) (width 0.2) (layer "F.Cu") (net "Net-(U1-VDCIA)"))
 (segment (start 90.98 52) (end 93.015 52) (width 0.2) (layer "F.Cu") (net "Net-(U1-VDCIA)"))
 (segment (start 94.775 50.24) (end 94.775 49.4625) (width 0.2) (layer "F.Cu") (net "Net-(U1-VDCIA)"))
 (segment (start 93.985 52) (end 95.175 50.81) (width 0.2) (layer "F.Cu") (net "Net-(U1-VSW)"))
 (segment (start 95.175 50.81) (end 95.175 49.4625) (width 0.2) (layer "F.Cu") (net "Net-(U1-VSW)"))
 (segment (start 95.975 49.4625) (end 95.975 50.154772) (width 0.2) (layer "F.Cu") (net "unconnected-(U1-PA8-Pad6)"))
 (segment (start 95.975 50.154772) (end 96.174999 50.354771) (width 0.2) (layer "F.Cu") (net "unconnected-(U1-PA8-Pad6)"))
 (via (at 96.174999 50.354771) (size 0.6) (drill 0.3) (layers "F.Cu" "B.Cu") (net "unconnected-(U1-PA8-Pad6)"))
 (segment (start 96.375 49.4625) (end 96.413019 49.4625) (width 0.2) (layer "F.Cu") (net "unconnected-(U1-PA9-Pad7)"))
 (segment (start 96.413019 49.4625) (end 96.715394 49.764875) (width 0.2) (layer "F.Cu") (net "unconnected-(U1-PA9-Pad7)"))
 (via (at 96.715394 49.764875) (size 0.6) (drill 0.3) (layers "F.Cu" "B.Cu") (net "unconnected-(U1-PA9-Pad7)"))
 (segment (start 93.975 45.5375) (end 91.121366 45.5375) (width 0.2) (layer "F.Cu") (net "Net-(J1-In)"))
 (segment (start 89.94 39.535) (end 89.975 39.5) (width 0.2) (layer "F.Cu") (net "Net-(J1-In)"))
 (segment (start 89.94 44.356134) (end 89.94 39.535) (width 0.2) (layer "F.Cu") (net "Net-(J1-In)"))
 (segment (start 91.121366 45.5375) (end 89.94 44.356134) (width 0.2) (layer "F.Cu") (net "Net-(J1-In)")))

